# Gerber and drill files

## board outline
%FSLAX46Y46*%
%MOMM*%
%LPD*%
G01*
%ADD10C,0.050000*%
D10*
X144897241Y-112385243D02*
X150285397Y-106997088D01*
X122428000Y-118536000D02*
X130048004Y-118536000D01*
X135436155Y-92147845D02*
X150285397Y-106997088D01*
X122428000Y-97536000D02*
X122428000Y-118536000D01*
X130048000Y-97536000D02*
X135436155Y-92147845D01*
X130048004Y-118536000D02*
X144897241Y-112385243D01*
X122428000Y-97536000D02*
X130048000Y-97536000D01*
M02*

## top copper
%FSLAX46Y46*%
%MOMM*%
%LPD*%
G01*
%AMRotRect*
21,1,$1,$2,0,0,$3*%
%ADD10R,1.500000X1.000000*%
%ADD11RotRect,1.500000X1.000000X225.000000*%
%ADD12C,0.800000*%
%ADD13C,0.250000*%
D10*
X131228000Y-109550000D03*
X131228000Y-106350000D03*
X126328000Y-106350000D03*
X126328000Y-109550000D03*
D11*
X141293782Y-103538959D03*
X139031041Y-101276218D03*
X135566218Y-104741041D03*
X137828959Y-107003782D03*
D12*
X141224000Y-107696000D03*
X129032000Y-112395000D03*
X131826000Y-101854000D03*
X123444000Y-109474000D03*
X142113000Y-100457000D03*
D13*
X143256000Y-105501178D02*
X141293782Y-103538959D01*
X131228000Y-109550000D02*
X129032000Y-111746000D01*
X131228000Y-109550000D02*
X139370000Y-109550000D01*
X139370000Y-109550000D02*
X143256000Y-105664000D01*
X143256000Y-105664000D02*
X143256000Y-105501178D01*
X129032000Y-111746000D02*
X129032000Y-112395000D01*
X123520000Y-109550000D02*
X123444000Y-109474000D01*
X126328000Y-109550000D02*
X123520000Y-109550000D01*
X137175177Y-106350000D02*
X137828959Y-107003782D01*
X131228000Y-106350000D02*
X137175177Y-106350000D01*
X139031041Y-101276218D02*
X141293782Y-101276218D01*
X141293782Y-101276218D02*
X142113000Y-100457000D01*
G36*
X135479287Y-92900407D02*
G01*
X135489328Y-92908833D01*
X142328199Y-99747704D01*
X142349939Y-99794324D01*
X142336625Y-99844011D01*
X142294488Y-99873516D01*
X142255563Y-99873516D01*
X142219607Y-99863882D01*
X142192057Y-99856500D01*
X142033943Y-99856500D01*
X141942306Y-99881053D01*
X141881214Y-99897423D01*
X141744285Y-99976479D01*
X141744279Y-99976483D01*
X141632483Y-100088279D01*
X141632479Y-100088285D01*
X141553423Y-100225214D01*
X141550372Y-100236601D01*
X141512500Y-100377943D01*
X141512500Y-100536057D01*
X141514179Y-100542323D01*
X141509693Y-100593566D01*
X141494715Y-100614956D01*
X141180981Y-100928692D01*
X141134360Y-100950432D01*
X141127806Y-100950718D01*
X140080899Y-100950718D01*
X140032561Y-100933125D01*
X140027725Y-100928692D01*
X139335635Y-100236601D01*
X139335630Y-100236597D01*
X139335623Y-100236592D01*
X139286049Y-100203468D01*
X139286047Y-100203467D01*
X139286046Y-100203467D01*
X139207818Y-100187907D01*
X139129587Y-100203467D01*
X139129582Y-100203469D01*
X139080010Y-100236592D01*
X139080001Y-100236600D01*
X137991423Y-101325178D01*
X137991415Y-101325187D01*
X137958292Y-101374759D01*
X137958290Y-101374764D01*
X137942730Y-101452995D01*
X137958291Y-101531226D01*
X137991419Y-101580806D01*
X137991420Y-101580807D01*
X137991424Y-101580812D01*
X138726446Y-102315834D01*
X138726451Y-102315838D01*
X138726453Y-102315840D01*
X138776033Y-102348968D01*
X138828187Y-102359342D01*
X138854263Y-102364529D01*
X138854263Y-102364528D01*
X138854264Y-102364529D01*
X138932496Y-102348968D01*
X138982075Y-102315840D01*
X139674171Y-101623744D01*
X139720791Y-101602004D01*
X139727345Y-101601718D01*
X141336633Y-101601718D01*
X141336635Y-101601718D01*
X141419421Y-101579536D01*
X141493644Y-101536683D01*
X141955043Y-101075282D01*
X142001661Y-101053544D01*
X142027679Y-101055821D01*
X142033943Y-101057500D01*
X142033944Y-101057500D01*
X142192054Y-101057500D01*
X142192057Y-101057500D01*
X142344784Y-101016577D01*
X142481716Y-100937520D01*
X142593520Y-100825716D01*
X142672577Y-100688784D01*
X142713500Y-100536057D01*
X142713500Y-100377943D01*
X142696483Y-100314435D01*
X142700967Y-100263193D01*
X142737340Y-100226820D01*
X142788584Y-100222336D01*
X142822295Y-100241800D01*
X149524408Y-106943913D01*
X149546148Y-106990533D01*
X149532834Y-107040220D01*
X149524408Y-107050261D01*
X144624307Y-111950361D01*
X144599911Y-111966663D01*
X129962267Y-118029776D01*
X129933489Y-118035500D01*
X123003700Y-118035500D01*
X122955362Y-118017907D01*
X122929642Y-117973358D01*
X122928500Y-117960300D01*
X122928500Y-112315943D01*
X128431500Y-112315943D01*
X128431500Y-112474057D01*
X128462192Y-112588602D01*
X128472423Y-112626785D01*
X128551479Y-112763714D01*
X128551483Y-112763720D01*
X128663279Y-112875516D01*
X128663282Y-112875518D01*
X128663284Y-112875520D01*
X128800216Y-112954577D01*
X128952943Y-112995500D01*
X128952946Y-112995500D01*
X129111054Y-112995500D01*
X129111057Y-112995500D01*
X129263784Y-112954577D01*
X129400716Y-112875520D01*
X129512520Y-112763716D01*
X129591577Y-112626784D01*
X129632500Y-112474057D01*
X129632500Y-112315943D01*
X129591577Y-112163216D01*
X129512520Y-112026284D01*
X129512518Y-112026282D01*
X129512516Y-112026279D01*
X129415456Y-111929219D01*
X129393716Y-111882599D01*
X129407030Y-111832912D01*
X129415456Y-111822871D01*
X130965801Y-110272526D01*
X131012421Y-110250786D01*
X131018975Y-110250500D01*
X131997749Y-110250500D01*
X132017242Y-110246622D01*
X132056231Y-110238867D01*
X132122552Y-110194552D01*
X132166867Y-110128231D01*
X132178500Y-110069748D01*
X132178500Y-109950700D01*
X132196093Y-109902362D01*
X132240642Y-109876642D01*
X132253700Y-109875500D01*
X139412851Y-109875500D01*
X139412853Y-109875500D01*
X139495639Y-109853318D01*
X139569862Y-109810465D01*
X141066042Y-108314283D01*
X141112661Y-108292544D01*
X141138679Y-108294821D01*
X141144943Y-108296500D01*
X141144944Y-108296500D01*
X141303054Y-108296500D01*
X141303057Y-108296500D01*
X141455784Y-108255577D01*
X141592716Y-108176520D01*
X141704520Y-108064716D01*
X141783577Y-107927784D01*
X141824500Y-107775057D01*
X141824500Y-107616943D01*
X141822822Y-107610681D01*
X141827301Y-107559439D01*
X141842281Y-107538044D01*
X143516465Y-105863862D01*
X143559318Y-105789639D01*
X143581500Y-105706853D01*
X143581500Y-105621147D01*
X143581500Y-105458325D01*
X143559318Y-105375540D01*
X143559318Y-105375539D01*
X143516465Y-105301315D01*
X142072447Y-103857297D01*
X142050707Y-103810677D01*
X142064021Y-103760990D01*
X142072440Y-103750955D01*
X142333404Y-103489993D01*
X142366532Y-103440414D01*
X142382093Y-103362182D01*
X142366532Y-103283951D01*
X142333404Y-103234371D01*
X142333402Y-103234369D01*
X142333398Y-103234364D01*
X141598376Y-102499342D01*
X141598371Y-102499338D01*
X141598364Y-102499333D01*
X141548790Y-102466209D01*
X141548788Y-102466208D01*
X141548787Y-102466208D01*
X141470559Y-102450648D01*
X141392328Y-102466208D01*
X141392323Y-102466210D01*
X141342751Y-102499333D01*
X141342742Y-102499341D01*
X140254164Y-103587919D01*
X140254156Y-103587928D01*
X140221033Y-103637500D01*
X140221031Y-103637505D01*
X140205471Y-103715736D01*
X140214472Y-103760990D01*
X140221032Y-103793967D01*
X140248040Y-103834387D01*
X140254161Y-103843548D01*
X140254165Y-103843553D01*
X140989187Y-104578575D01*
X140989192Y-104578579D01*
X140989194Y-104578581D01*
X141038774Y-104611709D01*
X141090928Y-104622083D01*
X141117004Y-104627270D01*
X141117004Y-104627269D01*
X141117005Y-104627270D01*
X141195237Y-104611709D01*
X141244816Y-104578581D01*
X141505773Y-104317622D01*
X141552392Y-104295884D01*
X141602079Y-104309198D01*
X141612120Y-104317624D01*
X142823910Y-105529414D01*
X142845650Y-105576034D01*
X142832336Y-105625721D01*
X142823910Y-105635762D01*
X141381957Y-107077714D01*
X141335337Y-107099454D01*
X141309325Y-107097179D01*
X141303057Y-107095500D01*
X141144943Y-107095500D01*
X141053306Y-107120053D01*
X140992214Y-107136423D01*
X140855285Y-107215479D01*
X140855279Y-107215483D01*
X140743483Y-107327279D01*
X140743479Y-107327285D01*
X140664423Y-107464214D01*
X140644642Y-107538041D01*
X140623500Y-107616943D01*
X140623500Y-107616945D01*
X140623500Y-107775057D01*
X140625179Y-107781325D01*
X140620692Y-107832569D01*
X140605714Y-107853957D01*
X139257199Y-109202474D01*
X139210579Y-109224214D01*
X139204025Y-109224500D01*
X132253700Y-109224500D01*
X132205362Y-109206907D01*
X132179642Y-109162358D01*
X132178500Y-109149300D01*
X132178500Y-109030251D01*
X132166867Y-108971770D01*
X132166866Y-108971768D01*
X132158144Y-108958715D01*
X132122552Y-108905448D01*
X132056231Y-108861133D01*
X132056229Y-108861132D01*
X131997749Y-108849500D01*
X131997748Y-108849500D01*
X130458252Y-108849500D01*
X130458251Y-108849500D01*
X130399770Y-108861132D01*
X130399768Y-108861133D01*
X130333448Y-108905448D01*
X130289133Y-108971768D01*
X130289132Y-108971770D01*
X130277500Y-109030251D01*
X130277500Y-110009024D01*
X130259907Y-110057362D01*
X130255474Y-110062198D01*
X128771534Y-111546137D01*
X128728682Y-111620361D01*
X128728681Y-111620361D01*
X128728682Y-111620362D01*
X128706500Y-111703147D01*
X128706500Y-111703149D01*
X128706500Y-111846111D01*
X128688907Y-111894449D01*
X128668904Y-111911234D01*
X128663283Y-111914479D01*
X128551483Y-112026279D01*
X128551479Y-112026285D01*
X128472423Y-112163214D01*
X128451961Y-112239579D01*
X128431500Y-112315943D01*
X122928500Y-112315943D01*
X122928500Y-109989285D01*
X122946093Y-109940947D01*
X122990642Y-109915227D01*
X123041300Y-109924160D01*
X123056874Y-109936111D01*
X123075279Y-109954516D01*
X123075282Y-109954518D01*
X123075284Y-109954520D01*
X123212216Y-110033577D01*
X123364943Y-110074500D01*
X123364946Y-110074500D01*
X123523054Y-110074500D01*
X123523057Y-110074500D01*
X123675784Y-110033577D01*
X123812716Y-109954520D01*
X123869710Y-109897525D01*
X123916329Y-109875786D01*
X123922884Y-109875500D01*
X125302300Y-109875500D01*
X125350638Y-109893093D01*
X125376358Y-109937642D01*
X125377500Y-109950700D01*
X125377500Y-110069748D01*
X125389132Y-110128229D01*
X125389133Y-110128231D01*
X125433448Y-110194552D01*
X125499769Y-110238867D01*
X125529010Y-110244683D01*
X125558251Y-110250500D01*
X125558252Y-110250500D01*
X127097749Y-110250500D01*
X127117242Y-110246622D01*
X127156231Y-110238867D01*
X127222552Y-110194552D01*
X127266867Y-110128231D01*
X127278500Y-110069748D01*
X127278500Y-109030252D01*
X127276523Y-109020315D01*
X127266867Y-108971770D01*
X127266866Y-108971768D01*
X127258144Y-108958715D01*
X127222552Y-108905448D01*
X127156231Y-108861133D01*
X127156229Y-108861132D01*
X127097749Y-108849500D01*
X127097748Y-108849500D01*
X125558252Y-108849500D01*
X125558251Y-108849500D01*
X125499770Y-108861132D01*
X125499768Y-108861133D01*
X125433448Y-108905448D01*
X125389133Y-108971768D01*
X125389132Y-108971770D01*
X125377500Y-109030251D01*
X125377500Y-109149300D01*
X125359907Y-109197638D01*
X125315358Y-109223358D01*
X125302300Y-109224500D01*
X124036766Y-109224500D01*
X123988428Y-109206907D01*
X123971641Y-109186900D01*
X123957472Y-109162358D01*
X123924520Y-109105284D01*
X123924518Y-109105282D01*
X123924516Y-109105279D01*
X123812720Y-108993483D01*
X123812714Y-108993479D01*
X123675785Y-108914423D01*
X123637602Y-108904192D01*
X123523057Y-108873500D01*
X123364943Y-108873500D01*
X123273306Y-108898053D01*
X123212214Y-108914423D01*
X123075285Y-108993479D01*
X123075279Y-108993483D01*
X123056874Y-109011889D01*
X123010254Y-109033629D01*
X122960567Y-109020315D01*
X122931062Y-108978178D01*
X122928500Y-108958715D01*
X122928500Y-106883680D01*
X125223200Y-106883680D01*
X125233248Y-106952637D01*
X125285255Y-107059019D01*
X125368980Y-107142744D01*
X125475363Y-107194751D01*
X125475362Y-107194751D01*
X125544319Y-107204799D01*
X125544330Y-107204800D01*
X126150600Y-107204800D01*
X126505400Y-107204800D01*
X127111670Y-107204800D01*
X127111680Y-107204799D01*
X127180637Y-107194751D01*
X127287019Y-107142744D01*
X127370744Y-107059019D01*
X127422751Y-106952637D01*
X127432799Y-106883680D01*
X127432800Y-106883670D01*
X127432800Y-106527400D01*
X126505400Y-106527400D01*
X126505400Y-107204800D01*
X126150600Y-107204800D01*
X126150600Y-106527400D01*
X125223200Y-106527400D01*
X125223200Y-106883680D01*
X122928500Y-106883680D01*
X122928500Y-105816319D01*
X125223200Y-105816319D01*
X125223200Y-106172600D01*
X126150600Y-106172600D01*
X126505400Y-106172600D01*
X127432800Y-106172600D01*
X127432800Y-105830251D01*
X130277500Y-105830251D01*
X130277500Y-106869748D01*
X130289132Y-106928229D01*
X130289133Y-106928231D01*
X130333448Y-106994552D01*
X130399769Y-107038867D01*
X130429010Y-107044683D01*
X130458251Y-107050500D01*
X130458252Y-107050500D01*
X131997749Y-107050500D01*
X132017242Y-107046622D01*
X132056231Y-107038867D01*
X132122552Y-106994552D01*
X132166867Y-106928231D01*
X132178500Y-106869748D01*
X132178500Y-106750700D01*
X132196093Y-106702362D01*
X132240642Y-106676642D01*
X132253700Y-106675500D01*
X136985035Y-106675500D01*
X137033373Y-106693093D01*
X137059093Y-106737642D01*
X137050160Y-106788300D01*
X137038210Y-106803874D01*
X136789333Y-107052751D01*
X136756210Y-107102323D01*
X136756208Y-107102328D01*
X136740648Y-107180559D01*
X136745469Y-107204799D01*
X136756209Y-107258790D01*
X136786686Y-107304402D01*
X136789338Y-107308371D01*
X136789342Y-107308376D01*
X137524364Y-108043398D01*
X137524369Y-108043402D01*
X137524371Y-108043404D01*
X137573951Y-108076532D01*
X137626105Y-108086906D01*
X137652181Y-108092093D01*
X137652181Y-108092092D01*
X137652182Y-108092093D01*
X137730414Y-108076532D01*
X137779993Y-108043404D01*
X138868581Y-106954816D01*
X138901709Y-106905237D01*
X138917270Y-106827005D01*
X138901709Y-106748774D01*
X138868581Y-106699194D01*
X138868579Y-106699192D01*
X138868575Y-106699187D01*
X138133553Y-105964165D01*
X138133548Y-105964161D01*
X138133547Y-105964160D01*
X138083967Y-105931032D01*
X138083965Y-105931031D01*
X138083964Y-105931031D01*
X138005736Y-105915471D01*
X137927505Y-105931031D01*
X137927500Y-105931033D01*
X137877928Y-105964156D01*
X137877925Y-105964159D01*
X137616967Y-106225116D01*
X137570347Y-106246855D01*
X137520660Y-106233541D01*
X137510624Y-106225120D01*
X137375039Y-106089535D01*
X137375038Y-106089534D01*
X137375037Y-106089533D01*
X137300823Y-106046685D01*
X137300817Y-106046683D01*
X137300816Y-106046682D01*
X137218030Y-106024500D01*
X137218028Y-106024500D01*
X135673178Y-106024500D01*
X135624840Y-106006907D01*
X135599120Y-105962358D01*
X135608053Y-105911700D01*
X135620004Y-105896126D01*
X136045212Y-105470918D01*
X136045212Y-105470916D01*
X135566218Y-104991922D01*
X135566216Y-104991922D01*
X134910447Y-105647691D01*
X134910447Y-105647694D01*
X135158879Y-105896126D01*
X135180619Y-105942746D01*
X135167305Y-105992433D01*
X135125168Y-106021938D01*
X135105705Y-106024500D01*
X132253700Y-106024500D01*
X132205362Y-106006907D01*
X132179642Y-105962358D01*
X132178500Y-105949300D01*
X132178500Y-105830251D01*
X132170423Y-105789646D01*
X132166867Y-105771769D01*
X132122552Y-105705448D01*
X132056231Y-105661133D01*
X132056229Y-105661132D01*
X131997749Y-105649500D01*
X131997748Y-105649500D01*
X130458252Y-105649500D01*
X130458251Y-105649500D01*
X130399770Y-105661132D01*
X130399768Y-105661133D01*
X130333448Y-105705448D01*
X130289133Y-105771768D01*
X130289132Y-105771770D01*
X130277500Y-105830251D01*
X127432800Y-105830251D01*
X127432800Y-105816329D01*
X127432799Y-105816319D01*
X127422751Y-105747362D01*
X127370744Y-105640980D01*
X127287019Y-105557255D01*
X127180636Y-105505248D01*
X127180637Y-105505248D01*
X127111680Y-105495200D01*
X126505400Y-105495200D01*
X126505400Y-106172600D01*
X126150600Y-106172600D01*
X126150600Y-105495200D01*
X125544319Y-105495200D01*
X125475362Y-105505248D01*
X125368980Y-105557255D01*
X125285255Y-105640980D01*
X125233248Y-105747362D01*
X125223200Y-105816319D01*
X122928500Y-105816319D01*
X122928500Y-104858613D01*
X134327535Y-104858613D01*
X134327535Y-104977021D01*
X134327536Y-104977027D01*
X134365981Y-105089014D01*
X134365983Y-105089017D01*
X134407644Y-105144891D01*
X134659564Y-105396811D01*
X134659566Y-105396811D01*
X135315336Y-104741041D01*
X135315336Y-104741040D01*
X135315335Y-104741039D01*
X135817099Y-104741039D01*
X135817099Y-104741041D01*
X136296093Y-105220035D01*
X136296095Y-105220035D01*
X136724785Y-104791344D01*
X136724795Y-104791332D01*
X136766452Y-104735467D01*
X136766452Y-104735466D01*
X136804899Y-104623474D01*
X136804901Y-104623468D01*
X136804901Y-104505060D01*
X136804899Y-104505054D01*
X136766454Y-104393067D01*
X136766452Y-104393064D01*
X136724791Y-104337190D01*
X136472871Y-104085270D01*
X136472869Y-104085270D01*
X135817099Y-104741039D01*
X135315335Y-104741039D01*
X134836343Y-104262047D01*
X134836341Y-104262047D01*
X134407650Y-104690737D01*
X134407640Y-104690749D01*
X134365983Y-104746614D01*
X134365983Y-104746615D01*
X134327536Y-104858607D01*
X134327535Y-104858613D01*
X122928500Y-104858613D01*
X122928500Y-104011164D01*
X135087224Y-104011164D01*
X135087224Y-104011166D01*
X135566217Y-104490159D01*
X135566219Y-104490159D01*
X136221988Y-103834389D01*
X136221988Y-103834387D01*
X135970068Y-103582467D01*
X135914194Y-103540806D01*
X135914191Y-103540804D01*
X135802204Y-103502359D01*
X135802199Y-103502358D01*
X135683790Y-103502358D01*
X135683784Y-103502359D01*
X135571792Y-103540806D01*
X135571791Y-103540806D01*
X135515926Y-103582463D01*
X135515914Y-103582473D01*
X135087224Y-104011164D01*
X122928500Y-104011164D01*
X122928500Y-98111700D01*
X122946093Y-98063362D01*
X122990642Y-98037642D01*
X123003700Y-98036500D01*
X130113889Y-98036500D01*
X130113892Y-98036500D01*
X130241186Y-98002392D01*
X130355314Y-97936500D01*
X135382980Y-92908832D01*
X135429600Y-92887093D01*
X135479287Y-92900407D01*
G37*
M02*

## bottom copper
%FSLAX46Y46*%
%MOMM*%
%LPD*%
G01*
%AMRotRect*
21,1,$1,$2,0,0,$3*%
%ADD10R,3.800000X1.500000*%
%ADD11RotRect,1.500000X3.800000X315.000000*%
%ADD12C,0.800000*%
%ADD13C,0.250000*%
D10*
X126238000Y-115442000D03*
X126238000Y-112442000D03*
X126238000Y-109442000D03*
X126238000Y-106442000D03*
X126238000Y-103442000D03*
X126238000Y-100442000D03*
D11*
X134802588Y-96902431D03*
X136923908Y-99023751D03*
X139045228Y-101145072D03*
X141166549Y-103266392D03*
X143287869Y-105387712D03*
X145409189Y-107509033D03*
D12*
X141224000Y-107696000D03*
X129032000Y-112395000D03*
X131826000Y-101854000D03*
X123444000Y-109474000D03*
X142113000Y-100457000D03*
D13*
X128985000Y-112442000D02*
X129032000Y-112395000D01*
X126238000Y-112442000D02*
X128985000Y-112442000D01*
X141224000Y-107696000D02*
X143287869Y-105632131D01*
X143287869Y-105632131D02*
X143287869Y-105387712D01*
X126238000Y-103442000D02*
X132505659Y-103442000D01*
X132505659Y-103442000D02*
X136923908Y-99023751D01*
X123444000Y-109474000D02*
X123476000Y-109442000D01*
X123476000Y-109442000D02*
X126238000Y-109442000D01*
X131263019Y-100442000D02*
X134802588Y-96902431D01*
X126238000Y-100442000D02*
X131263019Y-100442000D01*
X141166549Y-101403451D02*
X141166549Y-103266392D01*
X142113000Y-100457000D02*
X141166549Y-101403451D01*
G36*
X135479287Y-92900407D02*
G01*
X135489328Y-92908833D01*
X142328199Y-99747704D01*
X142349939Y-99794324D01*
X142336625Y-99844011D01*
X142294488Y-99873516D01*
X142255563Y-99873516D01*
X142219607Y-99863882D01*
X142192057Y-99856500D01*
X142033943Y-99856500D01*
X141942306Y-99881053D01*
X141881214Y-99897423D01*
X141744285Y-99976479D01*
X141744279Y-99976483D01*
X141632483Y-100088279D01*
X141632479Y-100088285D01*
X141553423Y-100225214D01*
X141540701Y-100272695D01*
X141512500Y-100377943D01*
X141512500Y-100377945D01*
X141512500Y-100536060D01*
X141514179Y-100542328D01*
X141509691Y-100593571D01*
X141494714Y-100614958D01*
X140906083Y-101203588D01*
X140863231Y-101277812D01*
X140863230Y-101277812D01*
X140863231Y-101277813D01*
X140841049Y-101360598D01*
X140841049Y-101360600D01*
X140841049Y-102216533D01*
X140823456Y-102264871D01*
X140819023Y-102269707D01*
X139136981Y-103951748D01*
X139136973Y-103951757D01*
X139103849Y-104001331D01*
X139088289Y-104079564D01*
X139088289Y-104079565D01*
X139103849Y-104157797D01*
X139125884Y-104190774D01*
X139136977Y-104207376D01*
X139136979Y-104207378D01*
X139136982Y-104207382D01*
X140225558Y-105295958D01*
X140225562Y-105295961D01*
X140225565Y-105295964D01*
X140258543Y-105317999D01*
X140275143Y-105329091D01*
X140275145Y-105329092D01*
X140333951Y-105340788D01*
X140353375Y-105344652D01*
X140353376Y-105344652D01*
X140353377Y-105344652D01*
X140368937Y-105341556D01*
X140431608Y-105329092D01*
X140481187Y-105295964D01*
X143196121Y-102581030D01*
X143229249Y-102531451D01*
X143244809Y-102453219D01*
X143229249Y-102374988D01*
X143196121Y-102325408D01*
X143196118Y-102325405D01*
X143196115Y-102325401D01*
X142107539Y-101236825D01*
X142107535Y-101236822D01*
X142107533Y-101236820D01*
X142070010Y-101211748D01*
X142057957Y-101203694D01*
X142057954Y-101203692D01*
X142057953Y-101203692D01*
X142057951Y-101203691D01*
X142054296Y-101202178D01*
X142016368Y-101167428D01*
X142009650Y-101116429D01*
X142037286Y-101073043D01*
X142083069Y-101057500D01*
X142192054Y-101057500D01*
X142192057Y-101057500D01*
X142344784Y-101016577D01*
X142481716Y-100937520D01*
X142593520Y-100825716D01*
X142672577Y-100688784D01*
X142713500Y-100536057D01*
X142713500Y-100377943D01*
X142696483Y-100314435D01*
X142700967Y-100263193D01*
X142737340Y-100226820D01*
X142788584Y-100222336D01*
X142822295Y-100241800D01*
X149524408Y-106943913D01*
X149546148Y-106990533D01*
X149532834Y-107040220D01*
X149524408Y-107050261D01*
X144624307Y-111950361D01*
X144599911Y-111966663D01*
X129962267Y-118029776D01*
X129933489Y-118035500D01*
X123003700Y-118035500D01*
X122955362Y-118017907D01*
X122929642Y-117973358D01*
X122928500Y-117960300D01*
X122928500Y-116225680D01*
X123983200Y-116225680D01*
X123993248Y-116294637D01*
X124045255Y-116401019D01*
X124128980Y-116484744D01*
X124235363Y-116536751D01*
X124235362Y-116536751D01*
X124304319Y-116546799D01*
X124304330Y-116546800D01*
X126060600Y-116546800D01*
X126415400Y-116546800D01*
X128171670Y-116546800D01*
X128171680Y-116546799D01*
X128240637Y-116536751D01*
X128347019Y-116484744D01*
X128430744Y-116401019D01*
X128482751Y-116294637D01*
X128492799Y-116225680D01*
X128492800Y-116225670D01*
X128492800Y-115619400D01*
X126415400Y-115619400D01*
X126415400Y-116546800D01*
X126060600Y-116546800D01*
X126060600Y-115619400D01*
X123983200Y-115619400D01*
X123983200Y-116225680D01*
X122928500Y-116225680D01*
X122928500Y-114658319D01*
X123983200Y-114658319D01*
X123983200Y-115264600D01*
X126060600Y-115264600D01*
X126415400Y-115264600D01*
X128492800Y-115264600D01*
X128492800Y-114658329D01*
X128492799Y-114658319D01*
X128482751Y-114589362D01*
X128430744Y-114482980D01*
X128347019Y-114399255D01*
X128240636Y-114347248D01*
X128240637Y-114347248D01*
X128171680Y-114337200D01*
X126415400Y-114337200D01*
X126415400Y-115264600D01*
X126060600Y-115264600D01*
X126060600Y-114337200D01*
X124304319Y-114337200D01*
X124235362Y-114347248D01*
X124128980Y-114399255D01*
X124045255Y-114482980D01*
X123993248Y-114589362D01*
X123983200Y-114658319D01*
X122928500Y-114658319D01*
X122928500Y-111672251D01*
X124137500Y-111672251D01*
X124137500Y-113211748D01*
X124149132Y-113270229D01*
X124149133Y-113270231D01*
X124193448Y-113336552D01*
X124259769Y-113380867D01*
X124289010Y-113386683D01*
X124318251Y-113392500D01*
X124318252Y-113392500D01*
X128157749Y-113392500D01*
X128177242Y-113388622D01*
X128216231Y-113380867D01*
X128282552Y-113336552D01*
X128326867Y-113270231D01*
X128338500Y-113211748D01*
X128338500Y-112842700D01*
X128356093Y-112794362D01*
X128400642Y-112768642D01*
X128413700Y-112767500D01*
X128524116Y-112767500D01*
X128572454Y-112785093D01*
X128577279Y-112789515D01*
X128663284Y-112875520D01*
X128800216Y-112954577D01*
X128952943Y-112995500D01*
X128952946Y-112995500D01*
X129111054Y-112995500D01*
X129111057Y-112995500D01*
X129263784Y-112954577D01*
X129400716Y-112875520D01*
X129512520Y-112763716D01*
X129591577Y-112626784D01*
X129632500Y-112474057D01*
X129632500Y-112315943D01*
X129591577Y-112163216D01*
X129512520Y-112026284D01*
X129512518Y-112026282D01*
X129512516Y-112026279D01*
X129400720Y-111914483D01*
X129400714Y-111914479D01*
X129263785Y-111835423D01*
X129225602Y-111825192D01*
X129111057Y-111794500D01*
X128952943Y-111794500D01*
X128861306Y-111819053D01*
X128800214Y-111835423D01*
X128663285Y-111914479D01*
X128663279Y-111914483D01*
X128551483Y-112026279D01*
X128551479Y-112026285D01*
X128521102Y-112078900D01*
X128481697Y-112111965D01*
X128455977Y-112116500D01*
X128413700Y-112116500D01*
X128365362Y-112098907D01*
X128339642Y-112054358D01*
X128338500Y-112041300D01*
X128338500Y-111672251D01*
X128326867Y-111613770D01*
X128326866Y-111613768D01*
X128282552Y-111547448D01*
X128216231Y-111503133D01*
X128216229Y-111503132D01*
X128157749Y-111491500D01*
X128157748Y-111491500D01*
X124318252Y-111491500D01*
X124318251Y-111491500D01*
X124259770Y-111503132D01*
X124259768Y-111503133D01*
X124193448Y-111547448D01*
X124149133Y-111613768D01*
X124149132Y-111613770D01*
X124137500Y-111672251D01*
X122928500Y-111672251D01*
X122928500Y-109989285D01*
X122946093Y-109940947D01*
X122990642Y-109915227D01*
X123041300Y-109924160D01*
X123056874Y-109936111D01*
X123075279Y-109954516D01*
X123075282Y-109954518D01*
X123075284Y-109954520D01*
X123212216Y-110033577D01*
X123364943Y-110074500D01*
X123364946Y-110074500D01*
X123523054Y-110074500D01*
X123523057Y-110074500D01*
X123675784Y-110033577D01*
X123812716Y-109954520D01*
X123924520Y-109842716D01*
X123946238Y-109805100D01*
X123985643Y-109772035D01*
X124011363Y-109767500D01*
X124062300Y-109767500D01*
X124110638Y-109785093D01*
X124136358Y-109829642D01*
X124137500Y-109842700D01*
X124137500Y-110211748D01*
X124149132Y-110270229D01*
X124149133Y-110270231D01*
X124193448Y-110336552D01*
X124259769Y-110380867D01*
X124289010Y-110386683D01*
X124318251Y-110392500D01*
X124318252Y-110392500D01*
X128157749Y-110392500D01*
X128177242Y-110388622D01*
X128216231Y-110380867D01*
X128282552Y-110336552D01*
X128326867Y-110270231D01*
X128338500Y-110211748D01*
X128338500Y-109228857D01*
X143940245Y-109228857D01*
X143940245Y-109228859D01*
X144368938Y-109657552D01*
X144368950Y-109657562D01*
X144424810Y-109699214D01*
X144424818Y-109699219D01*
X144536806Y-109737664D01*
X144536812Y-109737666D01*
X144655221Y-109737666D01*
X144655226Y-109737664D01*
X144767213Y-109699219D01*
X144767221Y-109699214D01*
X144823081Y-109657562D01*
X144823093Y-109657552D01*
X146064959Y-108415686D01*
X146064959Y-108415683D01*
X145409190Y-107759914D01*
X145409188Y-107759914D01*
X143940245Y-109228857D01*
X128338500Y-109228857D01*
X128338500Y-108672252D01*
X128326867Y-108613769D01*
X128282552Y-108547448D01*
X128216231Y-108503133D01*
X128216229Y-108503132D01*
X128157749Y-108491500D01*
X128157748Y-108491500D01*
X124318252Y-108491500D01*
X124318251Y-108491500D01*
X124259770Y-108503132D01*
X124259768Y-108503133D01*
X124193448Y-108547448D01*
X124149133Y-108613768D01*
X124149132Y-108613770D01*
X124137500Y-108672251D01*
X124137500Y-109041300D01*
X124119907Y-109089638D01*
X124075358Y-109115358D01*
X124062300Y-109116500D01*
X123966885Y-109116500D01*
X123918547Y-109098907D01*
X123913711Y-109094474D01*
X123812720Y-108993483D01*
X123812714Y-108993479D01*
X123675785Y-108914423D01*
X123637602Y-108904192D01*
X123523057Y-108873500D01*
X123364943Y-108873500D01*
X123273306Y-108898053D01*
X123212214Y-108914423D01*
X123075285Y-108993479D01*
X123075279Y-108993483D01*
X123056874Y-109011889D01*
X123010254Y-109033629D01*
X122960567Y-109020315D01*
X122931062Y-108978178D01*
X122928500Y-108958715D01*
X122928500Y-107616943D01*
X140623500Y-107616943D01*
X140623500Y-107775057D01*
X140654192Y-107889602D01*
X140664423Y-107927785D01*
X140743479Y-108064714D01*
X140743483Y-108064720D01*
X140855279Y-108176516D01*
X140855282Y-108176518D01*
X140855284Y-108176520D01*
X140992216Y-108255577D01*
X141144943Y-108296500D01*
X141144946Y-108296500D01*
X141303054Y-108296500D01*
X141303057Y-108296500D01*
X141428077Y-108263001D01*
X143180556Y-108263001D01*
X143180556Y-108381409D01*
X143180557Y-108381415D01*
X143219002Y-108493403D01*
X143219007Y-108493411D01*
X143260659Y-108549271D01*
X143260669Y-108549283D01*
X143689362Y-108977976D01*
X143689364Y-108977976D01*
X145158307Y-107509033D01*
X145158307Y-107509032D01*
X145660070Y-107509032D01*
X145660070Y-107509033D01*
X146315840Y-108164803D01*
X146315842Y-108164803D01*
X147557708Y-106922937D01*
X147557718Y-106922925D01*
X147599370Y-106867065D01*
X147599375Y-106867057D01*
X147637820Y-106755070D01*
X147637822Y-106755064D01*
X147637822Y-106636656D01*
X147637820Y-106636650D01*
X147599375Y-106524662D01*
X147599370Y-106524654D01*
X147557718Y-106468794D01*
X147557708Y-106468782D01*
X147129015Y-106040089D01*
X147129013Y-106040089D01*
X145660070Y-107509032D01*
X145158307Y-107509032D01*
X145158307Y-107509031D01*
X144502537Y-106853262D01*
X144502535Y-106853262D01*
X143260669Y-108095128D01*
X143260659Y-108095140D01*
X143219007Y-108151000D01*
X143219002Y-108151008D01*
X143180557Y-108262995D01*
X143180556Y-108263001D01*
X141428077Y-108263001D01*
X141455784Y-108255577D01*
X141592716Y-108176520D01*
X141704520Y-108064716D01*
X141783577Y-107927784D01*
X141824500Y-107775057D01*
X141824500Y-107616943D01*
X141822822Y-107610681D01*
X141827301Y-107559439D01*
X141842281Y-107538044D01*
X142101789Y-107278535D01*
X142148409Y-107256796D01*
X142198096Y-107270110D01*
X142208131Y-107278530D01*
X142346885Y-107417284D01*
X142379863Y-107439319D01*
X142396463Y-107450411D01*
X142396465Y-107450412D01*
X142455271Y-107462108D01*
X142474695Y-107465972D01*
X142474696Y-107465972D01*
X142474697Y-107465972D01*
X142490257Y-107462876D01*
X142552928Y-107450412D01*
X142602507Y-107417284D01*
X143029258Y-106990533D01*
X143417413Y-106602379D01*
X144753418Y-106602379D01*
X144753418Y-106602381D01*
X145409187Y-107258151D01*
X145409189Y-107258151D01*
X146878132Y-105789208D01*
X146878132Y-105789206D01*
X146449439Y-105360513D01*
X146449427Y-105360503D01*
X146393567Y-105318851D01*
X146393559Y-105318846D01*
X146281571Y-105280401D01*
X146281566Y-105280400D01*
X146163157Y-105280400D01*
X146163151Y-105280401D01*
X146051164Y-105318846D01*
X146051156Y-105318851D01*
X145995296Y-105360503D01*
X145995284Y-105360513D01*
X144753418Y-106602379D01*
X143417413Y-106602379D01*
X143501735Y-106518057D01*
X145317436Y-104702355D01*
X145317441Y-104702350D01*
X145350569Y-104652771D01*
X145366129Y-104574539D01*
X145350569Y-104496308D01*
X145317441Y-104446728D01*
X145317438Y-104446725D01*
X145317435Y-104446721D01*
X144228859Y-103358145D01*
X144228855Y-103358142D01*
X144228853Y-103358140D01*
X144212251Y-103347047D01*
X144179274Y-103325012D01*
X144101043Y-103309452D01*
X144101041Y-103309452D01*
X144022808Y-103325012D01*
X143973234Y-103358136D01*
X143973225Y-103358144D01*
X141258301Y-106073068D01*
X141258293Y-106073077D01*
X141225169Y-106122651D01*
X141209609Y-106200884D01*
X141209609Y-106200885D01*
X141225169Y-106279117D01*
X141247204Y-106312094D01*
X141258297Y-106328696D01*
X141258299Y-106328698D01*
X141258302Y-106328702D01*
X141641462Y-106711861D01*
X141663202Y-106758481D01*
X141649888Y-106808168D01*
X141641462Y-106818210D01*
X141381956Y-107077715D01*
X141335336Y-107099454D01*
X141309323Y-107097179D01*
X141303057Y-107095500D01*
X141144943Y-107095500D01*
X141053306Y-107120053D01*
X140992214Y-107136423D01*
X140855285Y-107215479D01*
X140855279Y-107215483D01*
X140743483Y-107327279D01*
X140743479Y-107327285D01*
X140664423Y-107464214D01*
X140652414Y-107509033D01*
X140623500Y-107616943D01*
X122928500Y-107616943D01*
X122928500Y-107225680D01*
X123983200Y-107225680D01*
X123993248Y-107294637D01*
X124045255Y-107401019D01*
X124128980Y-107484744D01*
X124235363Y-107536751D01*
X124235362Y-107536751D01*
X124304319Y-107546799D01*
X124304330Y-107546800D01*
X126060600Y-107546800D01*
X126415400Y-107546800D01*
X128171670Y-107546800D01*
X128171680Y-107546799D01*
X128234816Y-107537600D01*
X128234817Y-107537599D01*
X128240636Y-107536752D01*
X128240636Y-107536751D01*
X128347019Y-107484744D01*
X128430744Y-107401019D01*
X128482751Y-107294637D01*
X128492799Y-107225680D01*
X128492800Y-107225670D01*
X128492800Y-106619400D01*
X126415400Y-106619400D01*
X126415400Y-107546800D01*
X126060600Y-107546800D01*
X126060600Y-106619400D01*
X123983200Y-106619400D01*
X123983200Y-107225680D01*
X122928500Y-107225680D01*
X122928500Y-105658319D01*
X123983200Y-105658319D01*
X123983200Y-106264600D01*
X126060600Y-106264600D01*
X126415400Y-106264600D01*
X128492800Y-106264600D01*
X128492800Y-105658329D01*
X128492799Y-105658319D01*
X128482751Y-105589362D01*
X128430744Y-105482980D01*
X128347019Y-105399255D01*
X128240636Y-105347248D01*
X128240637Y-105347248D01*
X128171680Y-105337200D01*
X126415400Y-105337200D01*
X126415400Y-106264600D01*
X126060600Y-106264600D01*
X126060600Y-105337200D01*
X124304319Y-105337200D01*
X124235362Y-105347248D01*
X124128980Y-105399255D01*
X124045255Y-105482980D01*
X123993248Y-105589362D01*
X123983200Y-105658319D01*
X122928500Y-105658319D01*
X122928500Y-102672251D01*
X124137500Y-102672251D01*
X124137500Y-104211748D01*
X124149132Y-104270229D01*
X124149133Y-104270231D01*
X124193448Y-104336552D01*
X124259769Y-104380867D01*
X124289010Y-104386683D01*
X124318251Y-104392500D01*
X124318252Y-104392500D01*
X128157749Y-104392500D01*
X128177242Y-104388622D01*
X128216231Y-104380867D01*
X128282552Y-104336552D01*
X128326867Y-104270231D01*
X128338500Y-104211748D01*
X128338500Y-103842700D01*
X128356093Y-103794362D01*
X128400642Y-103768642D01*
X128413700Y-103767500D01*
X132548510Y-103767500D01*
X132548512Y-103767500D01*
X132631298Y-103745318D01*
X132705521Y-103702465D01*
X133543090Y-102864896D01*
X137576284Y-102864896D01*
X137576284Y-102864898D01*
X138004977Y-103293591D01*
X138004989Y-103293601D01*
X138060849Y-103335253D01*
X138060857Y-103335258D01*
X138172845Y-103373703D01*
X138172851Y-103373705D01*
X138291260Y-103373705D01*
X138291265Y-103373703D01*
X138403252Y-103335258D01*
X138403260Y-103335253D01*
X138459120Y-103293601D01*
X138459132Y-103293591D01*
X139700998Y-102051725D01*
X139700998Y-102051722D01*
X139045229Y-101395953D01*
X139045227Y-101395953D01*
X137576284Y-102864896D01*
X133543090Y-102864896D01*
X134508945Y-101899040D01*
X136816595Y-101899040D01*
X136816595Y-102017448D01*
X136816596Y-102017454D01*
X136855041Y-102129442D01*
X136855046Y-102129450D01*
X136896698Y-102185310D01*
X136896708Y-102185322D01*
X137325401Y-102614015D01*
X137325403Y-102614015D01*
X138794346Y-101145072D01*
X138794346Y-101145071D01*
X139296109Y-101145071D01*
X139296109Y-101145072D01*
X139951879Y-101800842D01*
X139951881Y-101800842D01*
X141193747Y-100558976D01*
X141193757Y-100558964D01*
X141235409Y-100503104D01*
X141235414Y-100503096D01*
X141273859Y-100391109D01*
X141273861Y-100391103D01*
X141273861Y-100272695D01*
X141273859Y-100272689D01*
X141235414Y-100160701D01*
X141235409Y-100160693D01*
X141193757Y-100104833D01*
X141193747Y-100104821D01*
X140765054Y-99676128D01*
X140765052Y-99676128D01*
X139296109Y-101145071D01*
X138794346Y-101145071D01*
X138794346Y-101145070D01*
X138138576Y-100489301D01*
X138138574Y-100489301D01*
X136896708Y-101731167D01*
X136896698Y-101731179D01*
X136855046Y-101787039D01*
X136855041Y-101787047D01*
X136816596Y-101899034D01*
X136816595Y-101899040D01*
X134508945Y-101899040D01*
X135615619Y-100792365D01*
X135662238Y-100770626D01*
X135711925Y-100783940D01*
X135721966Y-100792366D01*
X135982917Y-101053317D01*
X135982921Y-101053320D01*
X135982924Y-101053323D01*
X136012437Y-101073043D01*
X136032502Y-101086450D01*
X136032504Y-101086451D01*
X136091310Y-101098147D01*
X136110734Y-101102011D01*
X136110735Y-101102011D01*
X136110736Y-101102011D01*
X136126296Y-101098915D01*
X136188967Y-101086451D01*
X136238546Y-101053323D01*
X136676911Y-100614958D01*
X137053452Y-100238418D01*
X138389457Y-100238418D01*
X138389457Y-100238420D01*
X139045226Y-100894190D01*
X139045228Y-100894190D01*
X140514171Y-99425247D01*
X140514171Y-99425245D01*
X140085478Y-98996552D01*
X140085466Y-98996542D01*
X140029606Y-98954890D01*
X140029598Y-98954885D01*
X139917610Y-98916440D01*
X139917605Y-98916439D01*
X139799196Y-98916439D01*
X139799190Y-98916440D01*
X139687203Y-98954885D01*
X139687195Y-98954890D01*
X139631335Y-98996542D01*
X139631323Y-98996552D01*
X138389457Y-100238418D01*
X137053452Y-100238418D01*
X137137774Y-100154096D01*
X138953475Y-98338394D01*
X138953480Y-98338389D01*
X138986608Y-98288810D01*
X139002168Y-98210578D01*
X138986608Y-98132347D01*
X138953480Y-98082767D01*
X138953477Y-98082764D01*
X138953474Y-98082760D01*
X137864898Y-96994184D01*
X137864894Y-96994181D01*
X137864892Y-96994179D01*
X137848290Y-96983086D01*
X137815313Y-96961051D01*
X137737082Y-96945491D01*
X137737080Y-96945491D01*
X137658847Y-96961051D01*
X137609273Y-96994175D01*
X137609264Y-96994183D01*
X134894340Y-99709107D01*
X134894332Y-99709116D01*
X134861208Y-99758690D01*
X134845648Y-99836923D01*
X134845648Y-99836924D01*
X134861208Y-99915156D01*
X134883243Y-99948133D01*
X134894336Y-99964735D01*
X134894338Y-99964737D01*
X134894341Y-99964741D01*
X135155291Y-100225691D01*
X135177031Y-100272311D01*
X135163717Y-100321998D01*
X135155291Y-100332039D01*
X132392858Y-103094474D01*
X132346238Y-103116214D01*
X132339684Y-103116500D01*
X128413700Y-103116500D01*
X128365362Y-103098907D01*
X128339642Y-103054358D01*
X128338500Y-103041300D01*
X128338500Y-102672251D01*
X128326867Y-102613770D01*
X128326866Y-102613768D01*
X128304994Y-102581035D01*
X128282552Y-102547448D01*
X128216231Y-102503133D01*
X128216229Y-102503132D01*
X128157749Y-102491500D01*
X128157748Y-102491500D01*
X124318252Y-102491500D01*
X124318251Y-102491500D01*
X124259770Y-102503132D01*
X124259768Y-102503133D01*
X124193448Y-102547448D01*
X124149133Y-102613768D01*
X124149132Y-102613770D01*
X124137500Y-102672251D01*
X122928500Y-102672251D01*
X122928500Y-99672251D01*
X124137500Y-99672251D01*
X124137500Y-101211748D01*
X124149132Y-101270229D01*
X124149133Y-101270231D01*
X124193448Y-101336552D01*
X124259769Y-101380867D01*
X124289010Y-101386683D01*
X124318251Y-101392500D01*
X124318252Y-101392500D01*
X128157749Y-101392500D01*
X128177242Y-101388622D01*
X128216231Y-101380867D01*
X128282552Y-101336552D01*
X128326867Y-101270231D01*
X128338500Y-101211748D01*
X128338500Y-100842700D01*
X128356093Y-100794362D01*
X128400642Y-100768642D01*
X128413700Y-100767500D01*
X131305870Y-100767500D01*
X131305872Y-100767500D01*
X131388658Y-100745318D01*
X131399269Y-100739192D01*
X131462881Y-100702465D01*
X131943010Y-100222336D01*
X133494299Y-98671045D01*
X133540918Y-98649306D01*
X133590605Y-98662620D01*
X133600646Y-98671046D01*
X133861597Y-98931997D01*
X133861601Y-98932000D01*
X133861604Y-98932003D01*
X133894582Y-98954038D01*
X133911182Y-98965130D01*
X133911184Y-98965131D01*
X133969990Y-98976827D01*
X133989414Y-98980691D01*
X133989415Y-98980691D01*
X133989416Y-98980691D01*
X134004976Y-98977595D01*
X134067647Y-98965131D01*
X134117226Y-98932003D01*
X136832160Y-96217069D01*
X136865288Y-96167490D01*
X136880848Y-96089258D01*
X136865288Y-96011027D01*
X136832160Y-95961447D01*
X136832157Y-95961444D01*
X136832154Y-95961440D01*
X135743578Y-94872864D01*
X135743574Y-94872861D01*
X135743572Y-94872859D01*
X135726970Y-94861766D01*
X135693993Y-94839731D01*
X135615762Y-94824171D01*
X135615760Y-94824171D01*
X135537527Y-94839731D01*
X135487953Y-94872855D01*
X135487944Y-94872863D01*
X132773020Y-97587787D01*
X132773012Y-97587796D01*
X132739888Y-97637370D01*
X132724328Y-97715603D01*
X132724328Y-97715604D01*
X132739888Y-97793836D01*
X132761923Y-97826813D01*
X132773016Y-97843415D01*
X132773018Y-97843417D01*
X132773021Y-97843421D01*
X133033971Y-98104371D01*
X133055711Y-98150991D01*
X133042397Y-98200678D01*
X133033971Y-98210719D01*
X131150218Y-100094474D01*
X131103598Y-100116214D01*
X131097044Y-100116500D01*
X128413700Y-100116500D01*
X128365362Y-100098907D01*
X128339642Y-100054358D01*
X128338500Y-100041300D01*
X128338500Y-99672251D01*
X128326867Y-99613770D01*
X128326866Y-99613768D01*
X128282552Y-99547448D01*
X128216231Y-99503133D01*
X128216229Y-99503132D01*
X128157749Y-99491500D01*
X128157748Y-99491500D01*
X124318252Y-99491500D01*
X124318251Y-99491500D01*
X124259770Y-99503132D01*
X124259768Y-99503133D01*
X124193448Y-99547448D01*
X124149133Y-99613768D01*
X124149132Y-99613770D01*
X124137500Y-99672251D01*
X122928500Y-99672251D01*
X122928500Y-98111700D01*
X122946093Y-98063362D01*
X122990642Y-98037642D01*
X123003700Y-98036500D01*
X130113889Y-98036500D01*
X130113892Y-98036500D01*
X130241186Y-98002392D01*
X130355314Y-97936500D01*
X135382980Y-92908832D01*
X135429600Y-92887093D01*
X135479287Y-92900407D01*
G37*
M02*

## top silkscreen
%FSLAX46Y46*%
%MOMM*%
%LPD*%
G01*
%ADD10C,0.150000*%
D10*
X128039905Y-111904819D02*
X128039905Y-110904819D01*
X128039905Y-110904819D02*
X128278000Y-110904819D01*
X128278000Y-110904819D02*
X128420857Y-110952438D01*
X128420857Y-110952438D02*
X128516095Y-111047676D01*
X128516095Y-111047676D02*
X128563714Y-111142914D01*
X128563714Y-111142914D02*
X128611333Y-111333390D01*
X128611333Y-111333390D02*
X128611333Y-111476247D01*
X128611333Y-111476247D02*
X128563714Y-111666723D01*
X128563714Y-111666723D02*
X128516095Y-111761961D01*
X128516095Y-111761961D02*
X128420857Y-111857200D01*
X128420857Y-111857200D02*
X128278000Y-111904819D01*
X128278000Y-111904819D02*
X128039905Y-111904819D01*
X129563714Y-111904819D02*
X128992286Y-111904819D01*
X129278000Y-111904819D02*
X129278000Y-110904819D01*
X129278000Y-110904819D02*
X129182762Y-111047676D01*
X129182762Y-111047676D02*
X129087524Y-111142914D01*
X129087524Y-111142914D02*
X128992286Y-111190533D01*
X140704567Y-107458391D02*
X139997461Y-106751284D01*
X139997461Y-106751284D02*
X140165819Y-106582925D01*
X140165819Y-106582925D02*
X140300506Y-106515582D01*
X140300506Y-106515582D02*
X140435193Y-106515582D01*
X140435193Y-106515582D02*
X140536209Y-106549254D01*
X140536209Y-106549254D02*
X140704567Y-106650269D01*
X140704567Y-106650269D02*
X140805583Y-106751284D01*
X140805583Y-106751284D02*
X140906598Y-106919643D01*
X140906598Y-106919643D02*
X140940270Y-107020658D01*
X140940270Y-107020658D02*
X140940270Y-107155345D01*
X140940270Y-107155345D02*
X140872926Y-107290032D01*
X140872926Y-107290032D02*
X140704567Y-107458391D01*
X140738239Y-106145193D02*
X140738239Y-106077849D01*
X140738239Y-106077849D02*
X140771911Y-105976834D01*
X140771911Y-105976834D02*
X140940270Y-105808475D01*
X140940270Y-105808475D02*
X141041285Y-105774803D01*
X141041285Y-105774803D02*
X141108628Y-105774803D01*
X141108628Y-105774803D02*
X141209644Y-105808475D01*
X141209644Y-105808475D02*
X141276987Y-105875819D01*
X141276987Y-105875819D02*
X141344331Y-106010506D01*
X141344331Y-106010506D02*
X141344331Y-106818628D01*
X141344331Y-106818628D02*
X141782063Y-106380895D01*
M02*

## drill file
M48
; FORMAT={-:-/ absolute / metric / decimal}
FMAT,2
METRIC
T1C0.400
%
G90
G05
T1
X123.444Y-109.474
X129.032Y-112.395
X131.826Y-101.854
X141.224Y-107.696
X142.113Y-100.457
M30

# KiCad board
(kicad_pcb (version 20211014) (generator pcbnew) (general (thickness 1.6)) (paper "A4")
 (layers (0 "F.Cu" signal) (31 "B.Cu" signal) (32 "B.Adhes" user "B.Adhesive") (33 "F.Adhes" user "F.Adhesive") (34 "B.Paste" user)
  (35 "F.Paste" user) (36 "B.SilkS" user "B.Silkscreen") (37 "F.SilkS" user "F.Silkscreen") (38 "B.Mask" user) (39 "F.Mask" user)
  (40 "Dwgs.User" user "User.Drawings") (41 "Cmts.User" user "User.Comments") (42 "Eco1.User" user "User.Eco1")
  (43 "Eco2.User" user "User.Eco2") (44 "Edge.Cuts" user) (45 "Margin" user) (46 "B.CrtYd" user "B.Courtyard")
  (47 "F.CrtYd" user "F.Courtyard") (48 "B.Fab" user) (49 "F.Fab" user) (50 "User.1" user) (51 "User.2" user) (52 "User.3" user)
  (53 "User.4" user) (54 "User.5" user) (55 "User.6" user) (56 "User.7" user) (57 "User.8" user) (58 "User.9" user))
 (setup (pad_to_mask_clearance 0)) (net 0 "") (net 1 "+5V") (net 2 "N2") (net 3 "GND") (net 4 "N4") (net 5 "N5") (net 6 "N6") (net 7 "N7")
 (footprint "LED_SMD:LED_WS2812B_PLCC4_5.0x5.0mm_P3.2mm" (layer "F.Cu") (at 128.778 107.95 180)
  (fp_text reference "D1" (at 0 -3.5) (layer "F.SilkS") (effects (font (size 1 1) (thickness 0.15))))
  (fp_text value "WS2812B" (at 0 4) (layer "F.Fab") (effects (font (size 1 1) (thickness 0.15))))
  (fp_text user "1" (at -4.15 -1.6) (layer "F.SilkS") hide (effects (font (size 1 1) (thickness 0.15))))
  (pad "1" smd rect (at -2.45 -1.6 180) (size 1.5 1) (layers "F.Cu" "F.Paste" "F.Mask") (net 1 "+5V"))
  (pad "2" smd rect (at -2.45 1.6 180) (size 1.5 1) (layers "F.Cu" "F.Paste" "F.Mask") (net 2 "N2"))
  (pad "3" smd rect (at 2.45 1.6 180) (size 1.5 1) (layers "F.Cu" "F.Paste" "F.Mask") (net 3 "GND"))
  (pad "4" smd rect (at 2.45 -1.6 180) (size 1.5 1) (layers "F.Cu" "F.Paste" "F.Mask") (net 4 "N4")))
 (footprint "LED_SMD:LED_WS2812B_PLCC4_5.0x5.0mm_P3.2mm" (layer "F.Cu") (at 138.43 104.14 -135)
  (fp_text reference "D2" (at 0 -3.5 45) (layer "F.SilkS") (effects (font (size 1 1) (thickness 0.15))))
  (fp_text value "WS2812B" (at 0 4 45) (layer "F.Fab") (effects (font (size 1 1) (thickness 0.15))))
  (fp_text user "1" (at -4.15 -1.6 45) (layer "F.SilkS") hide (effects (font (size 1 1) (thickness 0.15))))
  (pad "1" smd rect (at -2.45 -1.6 225) (size 1.5 1) (layers "F.Cu" "F.Paste" "F.Mask") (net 1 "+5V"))
  (pad "2" smd rect (at -2.45 1.6 225) (size 1.5 1) (layers "F.Cu" "F.Paste" "F.Mask") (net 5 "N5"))
  (pad "3" smd rect (at 2.45 1.6 225) (size 1.5 1) (layers "F.Cu" "F.Paste" "F.Mask") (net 3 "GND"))
  (pad "4" smd rect (at 2.45 -1.6 225) (size 1.5 1) (layers "F.Cu" "F.Paste" "F.Mask") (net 2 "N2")))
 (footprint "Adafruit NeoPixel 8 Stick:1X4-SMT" (layer "B.Cu") (at 126.873 107.442 90)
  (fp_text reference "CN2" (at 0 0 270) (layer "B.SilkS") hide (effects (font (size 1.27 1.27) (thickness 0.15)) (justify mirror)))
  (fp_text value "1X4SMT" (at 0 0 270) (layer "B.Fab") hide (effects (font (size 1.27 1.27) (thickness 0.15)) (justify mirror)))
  (pad "1" smd rect (at -8 -0.635 90) (size 1.5 3.8) (layers "B.Cu" "B.Paste" "B.Mask") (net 3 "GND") (solder_mask_margin 0.1016))
  (pad "2" smd rect (at -5 -0.635 90) (size 1.5 3.8) (layers "B.Cu" "B.Paste" "B.Mask") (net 1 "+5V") (solder_mask_margin 0.1016))
  (pad "3" smd rect (at -2 -0.635 90) (size 1.5 3.8) (layers "B.Cu" "B.Paste" "B.Mask") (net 4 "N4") (solder_mask_margin 0.1016))
  (pad "4" smd rect (at 1 -0.635 90) (size 1.5 3.8) (layers "B.Cu" "B.Paste" "B.Mask") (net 3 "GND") (solder_mask_margin 0.1016))
  (pad "5" smd rect (at 4 -0.635 90) (size 1.5 3.8) (layers "B.Cu" "B.Paste" "B.Mask") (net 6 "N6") (solder_mask_margin 0.1016))
  (pad "6" smd rect (at 7 -0.635 90) (size 1.5 3.8) (layers "B.Cu" "B.Paste" "B.Mask") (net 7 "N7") (solder_mask_margin 0.1016)))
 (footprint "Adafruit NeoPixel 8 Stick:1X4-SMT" (layer "B.Cu") (at 140.010429 103.008298 -45)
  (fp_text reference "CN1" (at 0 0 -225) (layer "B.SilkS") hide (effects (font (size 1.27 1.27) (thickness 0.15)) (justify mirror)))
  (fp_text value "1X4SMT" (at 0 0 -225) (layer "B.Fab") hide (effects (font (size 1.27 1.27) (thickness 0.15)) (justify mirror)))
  (pad "1" smd rect (at -8 -0.635 315) (size 1.5 3.8) (layers "B.Cu" "B.Paste" "B.Mask") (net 7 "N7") (solder_mask_margin 0.1016))
  (pad "2" smd rect (at -5 -0.635 315) (size 1.5 3.8) (layers "B.Cu" "B.Paste" "B.Mask") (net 6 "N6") (solder_mask_margin 0.1016))
  (pad "3" smd rect (at -2 -0.635 315) (size 1.5 3.8) (layers "B.Cu" "B.Paste" "B.Mask") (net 3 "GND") (solder_mask_margin 0.1016))
  (pad "4" smd rect (at 1 -0.635 315) (size 1.5 3.8) (layers "B.Cu" "B.Paste" "B.Mask") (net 5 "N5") (solder_mask_margin 0.1016))
  (pad "5" smd rect (at 4 -0.635 315) (size 1.5 3.8) (layers "B.Cu" "B.Paste" "B.Mask") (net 1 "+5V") (solder_mask_margin 0.1016))
  (pad "6" smd rect (at 7 -0.635 315) (size 1.5 3.8) (layers "B.Cu" "B.Paste" "B.Mask") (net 3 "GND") (solder_mask_margin 0.1016)))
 (gr_line locked (start 144.897241 112.385243) (end 150.285397 106.997088) (layer "Edge.Cuts") (width 0.05))
 (gr_line (start 122.428 118.536) (end 130.048004 118.536) (layer "Edge.Cuts") (width 0.05))
 (gr_line (start 135.436155 92.147845) (end 150.285397 106.997088) (layer "Edge.Cuts") (width 0.05))
 (gr_line (start 122.428 97.536) (end 122.428 118.536) (layer "Edge.Cuts") (width 0.05))
 (gr_line (start 130.048 97.536) (end 135.436155 92.147845) (layer "Edge.Cuts") (width 0.05))
 (gr_line (start 130.048004 118.536) (end 144.897241 112.385243) (layer "Edge.Cuts") (width 0.05))
 (gr_line (start 122.428 97.536) (end 130.048 97.536) (layer "Edge.Cuts") (width 0.05))
 (segment (start 143.256 105.501178) (end 141.293782 103.538959) (width 0.25) (layer "F.Cu") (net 1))
 (segment (start 131.228 109.55) (end 129.032 111.746) (width 0.25) (layer "F.Cu") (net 1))
 (segment (start 131.228 109.55) (end 139.37 109.55) (width 0.25) (layer "F.Cu") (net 1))
 (segment (start 139.37 109.55) (end 143.256 105.664) (width 0.25) (layer "F.Cu") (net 1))
 (segment (start 143.256 105.664) (end 143.256 105.501178) (width 0.25) (layer "F.Cu") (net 1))
 (segment (start 129.032 111.746) (end 129.032 112.395) (width 0.25) (layer "F.Cu") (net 1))
 (via (at 141.224 107.696) (size 0.8) (drill 0.4) (layers "F.Cu" "B.Cu") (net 1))
 (via (at 129.032 112.395) (size 0.8) (drill 0.4) (layers "F.Cu" "B.Cu") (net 1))
 (segment (start 128.985 112.442) (end 129.032 112.395) (width 0.25) (layer "B.Cu") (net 1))
 (segment (start 126.238 112.442) (end 128.985 112.442) (width 0.25) (layer "B.Cu") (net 1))
 (segment (start 141.224 107.696) (end 143.287869 105.632131) (width 0.25) (layer "B.Cu") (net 1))
 (segment (start 143.287869 105.632131) (end 143.287869 105.387712) (width 0.25) (layer "B.Cu") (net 1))
 (via (at 131.826 101.854) (size 0.8) (drill 0.4) (layers "F.Cu" "B.Cu") (free) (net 3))
 (segment (start 126.238 103.442) (end 132.505659 103.442) (width 0.25) (layer "B.Cu") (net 6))
 (segment (start 132.505659 103.442) (end 136.923908 99.023751) (width 0.25) (layer "B.Cu") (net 6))
 (segment (start 123.52 109.55) (end 123.444 109.474) (width 0.25) (layer "F.Cu") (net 4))
 (segment (start 126.328 109.55) (end 123.52 109.55) (width 0.25) (layer "F.Cu") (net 4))
 (via (at 123.444 109.474) (size 0.8) (drill 0.4) (layers "F.Cu" "B.Cu") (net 4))
 (segment (start 123.444 109.474) (end 123.476 109.442) (width 0.25) (layer "B.Cu") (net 4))
 (segment (start 123.476 109.442) (end 126.238 109.442) (width 0.25) (layer "B.Cu") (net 4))
 (segment (start 137.175177 106.35) (end 137.828959 107.003782) (width 0.25) (layer "F.Cu") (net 2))
 (segment (start 131.228 106.35) (end 137.175177 106.35) (width 0.25) (layer "F.Cu") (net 2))
 (segment (start 131.263019 100.442) (end 134.802588 96.902431) (width 0.25) (layer "B.Cu") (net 7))
 (segment (start 126.238 100.442) (end 131.263019 100.442) (width 0.25) (layer "B.Cu") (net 7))
 (segment (start 139.031041 101.276218) (end 141.293782 101.276218) (width 0.25) (layer "F.Cu") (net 5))
 (segment (start 141.293782 101.276218) (end 142.113 100.457) (width 0.25) (layer "F.Cu") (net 5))
 (via (at 142.113 100.457) (size 0.8) (drill 0.4) (layers "F.Cu" "B.Cu") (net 5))
 (segment (start 141.166549 101.403451) (end 141.166549 103.266392) (width 0.25) (layer "B.Cu") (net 5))
 (segment (start 142.113 100.457) (end 141.166549 101.403451) (width 0.25) (layer "B.Cu") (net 5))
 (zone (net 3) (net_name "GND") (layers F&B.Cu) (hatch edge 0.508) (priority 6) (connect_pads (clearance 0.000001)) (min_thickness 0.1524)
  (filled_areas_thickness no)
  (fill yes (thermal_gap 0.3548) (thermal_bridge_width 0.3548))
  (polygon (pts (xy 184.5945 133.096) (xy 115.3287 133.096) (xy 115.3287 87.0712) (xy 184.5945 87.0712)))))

